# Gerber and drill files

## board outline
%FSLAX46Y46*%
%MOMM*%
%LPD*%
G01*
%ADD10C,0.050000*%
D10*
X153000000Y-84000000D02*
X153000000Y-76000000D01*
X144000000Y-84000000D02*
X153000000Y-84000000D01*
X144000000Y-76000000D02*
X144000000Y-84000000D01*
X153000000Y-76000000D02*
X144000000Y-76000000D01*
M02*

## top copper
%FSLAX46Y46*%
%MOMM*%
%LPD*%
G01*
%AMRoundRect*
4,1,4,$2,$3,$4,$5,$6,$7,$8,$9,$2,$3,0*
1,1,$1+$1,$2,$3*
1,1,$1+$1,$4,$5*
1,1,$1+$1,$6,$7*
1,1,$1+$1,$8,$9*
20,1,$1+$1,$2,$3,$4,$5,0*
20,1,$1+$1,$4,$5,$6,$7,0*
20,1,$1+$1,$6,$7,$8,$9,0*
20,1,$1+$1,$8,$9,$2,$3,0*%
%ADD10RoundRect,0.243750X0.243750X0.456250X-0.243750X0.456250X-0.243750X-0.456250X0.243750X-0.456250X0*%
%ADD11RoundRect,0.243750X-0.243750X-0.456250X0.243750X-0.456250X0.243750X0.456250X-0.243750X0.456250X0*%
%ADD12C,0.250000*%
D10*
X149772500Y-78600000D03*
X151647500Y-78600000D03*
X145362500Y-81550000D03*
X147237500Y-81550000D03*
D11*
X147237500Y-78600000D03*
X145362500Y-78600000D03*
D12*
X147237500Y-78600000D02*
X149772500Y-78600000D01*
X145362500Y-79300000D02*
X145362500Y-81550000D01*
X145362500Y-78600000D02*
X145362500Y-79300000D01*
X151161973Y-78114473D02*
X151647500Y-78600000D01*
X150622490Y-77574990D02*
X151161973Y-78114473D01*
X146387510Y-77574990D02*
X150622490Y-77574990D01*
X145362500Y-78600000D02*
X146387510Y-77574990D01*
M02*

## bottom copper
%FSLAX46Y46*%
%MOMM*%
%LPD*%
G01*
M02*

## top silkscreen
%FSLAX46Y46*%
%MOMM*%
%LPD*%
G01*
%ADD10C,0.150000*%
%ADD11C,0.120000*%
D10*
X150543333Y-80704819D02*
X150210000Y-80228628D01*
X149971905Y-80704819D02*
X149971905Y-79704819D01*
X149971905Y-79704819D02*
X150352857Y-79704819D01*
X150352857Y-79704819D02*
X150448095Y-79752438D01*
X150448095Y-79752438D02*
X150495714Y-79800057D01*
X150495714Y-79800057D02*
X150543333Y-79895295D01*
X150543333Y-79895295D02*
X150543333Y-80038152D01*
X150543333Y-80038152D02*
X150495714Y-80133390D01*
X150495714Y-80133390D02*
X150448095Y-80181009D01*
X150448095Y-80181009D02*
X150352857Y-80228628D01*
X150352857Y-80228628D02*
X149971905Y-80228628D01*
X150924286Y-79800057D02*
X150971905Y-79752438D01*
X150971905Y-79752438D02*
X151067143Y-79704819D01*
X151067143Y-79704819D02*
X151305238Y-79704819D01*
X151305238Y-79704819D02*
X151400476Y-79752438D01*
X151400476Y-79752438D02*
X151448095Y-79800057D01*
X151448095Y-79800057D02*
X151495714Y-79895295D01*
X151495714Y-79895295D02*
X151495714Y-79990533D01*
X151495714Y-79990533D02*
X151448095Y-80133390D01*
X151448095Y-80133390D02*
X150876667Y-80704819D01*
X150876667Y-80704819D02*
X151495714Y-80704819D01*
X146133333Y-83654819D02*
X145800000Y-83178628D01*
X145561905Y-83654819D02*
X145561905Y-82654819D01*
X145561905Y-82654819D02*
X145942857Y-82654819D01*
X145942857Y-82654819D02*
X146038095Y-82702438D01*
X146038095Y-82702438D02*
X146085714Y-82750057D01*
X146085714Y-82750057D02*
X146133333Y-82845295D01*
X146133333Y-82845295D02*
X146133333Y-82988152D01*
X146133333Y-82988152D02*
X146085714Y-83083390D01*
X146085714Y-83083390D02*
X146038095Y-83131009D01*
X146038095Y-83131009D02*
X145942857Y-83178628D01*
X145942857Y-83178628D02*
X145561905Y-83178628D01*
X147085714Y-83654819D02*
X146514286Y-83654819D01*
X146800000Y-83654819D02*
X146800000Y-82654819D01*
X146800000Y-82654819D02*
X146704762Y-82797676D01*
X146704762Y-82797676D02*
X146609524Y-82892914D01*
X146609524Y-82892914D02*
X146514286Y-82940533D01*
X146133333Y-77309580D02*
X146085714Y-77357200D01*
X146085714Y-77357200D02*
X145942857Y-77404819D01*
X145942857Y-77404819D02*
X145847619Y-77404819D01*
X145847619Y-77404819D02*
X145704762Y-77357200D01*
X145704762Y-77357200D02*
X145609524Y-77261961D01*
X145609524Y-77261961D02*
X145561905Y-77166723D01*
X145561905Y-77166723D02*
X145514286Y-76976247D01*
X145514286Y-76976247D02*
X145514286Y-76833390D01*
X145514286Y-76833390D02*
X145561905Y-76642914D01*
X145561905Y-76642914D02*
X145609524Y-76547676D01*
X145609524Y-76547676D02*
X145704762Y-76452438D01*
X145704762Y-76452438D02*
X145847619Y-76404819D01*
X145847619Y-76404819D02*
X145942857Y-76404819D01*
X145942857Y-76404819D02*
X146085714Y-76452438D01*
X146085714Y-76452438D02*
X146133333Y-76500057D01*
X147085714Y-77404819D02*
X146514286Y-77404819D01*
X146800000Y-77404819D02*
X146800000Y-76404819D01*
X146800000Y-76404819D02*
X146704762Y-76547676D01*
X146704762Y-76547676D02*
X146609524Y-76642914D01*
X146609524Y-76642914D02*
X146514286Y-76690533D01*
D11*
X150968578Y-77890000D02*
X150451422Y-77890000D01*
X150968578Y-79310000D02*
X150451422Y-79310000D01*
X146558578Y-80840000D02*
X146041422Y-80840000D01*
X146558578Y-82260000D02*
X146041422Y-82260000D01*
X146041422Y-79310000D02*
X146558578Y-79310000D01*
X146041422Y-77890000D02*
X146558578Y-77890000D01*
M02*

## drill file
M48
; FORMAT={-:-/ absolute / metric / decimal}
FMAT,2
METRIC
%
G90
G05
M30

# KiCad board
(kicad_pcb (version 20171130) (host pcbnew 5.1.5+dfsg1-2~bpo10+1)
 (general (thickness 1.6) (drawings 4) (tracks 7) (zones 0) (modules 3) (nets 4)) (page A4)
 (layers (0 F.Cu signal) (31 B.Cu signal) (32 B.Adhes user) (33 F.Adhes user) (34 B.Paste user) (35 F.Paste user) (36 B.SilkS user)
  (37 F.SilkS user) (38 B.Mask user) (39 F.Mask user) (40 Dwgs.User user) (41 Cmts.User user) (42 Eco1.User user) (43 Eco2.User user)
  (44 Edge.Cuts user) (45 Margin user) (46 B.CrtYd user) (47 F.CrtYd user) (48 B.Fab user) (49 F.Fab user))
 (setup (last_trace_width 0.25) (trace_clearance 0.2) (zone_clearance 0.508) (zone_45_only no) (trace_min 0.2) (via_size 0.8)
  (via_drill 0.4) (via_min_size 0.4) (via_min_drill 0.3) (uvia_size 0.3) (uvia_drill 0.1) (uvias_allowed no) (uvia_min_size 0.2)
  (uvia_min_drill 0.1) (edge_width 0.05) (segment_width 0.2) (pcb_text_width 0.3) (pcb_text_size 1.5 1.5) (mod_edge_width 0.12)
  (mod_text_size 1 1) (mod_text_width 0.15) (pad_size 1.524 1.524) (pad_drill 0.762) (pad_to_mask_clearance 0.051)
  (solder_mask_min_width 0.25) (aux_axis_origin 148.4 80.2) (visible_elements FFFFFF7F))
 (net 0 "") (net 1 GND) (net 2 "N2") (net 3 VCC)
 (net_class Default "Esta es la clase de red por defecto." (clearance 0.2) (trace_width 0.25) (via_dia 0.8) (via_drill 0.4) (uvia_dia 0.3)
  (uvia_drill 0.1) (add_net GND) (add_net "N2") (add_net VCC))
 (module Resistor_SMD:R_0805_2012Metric (layer F.Cu) (at 150.71 78.6 180)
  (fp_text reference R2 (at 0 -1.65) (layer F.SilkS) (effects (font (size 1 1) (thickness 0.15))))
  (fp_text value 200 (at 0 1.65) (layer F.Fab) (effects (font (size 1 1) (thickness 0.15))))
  (fp_line (start -0.258578 0.71) (end 0.258578 0.71) (layer F.SilkS) (width 0.12))
  (fp_line (start -0.258578 -0.71) (end 0.258578 -0.71) (layer F.SilkS) (width 0.12))
  (pad 2 smd roundrect (at 0.9375 0 180) (size 0.975 1.4) (layers F.Cu F.Paste F.Mask) (roundrect_rratio 0.25) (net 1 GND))
  (pad 1 smd roundrect (at -0.9375 0 180) (size 0.975 1.4) (layers F.Cu F.Paste F.Mask) (roundrect_rratio 0.25) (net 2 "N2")))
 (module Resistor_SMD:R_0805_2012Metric (layer F.Cu) (at 146.3 81.55 180)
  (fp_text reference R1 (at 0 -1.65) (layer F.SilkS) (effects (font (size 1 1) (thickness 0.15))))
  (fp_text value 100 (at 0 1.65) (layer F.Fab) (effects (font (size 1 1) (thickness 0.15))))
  (fp_line (start -0.258578 0.71) (end 0.258578 0.71) (layer F.SilkS) (width 0.12))
  (fp_line (start -0.258578 -0.71) (end 0.258578 -0.71) (layer F.SilkS) (width 0.12))
  (pad 2 smd roundrect (at 0.9375 0 180) (size 0.975 1.4) (layers F.Cu F.Paste F.Mask) (roundrect_rratio 0.25) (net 2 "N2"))
  (pad 1 smd roundrect (at -0.9375 0 180) (size 0.975 1.4) (layers F.Cu F.Paste F.Mask) (roundrect_rratio 0.25) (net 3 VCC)))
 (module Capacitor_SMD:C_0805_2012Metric (layer F.Cu) (at 146.3 78.6)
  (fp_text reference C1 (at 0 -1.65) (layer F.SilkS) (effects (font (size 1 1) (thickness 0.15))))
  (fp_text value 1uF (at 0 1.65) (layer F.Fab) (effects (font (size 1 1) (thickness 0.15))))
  (fp_line (start -0.258578 0.71) (end 0.258578 0.71) (layer F.SilkS) (width 0.12))
  (fp_line (start -0.258578 -0.71) (end 0.258578 -0.71) (layer F.SilkS) (width 0.12))
  (pad 2 smd roundrect (at 0.9375 0) (size 0.975 1.4) (layers F.Cu F.Paste F.Mask) (roundrect_rratio 0.25) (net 1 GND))
  (pad 1 smd roundrect (at -0.9375 0) (size 0.975 1.4) (layers F.Cu F.Paste F.Mask) (roundrect_rratio 0.25) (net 2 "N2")))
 (gr_line (start 153 84) (end 153 76) (layer Edge.Cuts) (width 0.05))
 (gr_line (start 144 84) (end 153 84) (layer Edge.Cuts) (width 0.05))
 (gr_line (start 144 76) (end 144 84) (layer Edge.Cuts) (width 0.05))
 (gr_line (start 153 76) (end 144 76) (layer Edge.Cuts) (width 0.05))
 (segment (start 147.2375 78.6) (end 149.7725 78.6) (width 0.25) (layer F.Cu) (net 1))
 (segment (start 145.3625 79.3) (end 145.3625 81.55) (width 0.25) (layer F.Cu) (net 2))
 (segment (start 145.3625 78.6) (end 145.3625 79.3) (width 0.25) (layer F.Cu) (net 2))
 (segment (start 151.161973 78.114473) (end 151.6475 78.6) (width 0.25) (layer F.Cu) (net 2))
 (segment (start 150.62249 77.57499) (end 151.161973 78.114473) (width 0.25) (layer F.Cu) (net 2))
 (segment (start 146.38751 77.57499) (end 150.62249 77.57499) (width 0.25) (layer F.Cu) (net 2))
 (segment (start 145.3625 78.6) (end 146.38751 77.57499) (width 0.25) (layer F.Cu) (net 2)))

